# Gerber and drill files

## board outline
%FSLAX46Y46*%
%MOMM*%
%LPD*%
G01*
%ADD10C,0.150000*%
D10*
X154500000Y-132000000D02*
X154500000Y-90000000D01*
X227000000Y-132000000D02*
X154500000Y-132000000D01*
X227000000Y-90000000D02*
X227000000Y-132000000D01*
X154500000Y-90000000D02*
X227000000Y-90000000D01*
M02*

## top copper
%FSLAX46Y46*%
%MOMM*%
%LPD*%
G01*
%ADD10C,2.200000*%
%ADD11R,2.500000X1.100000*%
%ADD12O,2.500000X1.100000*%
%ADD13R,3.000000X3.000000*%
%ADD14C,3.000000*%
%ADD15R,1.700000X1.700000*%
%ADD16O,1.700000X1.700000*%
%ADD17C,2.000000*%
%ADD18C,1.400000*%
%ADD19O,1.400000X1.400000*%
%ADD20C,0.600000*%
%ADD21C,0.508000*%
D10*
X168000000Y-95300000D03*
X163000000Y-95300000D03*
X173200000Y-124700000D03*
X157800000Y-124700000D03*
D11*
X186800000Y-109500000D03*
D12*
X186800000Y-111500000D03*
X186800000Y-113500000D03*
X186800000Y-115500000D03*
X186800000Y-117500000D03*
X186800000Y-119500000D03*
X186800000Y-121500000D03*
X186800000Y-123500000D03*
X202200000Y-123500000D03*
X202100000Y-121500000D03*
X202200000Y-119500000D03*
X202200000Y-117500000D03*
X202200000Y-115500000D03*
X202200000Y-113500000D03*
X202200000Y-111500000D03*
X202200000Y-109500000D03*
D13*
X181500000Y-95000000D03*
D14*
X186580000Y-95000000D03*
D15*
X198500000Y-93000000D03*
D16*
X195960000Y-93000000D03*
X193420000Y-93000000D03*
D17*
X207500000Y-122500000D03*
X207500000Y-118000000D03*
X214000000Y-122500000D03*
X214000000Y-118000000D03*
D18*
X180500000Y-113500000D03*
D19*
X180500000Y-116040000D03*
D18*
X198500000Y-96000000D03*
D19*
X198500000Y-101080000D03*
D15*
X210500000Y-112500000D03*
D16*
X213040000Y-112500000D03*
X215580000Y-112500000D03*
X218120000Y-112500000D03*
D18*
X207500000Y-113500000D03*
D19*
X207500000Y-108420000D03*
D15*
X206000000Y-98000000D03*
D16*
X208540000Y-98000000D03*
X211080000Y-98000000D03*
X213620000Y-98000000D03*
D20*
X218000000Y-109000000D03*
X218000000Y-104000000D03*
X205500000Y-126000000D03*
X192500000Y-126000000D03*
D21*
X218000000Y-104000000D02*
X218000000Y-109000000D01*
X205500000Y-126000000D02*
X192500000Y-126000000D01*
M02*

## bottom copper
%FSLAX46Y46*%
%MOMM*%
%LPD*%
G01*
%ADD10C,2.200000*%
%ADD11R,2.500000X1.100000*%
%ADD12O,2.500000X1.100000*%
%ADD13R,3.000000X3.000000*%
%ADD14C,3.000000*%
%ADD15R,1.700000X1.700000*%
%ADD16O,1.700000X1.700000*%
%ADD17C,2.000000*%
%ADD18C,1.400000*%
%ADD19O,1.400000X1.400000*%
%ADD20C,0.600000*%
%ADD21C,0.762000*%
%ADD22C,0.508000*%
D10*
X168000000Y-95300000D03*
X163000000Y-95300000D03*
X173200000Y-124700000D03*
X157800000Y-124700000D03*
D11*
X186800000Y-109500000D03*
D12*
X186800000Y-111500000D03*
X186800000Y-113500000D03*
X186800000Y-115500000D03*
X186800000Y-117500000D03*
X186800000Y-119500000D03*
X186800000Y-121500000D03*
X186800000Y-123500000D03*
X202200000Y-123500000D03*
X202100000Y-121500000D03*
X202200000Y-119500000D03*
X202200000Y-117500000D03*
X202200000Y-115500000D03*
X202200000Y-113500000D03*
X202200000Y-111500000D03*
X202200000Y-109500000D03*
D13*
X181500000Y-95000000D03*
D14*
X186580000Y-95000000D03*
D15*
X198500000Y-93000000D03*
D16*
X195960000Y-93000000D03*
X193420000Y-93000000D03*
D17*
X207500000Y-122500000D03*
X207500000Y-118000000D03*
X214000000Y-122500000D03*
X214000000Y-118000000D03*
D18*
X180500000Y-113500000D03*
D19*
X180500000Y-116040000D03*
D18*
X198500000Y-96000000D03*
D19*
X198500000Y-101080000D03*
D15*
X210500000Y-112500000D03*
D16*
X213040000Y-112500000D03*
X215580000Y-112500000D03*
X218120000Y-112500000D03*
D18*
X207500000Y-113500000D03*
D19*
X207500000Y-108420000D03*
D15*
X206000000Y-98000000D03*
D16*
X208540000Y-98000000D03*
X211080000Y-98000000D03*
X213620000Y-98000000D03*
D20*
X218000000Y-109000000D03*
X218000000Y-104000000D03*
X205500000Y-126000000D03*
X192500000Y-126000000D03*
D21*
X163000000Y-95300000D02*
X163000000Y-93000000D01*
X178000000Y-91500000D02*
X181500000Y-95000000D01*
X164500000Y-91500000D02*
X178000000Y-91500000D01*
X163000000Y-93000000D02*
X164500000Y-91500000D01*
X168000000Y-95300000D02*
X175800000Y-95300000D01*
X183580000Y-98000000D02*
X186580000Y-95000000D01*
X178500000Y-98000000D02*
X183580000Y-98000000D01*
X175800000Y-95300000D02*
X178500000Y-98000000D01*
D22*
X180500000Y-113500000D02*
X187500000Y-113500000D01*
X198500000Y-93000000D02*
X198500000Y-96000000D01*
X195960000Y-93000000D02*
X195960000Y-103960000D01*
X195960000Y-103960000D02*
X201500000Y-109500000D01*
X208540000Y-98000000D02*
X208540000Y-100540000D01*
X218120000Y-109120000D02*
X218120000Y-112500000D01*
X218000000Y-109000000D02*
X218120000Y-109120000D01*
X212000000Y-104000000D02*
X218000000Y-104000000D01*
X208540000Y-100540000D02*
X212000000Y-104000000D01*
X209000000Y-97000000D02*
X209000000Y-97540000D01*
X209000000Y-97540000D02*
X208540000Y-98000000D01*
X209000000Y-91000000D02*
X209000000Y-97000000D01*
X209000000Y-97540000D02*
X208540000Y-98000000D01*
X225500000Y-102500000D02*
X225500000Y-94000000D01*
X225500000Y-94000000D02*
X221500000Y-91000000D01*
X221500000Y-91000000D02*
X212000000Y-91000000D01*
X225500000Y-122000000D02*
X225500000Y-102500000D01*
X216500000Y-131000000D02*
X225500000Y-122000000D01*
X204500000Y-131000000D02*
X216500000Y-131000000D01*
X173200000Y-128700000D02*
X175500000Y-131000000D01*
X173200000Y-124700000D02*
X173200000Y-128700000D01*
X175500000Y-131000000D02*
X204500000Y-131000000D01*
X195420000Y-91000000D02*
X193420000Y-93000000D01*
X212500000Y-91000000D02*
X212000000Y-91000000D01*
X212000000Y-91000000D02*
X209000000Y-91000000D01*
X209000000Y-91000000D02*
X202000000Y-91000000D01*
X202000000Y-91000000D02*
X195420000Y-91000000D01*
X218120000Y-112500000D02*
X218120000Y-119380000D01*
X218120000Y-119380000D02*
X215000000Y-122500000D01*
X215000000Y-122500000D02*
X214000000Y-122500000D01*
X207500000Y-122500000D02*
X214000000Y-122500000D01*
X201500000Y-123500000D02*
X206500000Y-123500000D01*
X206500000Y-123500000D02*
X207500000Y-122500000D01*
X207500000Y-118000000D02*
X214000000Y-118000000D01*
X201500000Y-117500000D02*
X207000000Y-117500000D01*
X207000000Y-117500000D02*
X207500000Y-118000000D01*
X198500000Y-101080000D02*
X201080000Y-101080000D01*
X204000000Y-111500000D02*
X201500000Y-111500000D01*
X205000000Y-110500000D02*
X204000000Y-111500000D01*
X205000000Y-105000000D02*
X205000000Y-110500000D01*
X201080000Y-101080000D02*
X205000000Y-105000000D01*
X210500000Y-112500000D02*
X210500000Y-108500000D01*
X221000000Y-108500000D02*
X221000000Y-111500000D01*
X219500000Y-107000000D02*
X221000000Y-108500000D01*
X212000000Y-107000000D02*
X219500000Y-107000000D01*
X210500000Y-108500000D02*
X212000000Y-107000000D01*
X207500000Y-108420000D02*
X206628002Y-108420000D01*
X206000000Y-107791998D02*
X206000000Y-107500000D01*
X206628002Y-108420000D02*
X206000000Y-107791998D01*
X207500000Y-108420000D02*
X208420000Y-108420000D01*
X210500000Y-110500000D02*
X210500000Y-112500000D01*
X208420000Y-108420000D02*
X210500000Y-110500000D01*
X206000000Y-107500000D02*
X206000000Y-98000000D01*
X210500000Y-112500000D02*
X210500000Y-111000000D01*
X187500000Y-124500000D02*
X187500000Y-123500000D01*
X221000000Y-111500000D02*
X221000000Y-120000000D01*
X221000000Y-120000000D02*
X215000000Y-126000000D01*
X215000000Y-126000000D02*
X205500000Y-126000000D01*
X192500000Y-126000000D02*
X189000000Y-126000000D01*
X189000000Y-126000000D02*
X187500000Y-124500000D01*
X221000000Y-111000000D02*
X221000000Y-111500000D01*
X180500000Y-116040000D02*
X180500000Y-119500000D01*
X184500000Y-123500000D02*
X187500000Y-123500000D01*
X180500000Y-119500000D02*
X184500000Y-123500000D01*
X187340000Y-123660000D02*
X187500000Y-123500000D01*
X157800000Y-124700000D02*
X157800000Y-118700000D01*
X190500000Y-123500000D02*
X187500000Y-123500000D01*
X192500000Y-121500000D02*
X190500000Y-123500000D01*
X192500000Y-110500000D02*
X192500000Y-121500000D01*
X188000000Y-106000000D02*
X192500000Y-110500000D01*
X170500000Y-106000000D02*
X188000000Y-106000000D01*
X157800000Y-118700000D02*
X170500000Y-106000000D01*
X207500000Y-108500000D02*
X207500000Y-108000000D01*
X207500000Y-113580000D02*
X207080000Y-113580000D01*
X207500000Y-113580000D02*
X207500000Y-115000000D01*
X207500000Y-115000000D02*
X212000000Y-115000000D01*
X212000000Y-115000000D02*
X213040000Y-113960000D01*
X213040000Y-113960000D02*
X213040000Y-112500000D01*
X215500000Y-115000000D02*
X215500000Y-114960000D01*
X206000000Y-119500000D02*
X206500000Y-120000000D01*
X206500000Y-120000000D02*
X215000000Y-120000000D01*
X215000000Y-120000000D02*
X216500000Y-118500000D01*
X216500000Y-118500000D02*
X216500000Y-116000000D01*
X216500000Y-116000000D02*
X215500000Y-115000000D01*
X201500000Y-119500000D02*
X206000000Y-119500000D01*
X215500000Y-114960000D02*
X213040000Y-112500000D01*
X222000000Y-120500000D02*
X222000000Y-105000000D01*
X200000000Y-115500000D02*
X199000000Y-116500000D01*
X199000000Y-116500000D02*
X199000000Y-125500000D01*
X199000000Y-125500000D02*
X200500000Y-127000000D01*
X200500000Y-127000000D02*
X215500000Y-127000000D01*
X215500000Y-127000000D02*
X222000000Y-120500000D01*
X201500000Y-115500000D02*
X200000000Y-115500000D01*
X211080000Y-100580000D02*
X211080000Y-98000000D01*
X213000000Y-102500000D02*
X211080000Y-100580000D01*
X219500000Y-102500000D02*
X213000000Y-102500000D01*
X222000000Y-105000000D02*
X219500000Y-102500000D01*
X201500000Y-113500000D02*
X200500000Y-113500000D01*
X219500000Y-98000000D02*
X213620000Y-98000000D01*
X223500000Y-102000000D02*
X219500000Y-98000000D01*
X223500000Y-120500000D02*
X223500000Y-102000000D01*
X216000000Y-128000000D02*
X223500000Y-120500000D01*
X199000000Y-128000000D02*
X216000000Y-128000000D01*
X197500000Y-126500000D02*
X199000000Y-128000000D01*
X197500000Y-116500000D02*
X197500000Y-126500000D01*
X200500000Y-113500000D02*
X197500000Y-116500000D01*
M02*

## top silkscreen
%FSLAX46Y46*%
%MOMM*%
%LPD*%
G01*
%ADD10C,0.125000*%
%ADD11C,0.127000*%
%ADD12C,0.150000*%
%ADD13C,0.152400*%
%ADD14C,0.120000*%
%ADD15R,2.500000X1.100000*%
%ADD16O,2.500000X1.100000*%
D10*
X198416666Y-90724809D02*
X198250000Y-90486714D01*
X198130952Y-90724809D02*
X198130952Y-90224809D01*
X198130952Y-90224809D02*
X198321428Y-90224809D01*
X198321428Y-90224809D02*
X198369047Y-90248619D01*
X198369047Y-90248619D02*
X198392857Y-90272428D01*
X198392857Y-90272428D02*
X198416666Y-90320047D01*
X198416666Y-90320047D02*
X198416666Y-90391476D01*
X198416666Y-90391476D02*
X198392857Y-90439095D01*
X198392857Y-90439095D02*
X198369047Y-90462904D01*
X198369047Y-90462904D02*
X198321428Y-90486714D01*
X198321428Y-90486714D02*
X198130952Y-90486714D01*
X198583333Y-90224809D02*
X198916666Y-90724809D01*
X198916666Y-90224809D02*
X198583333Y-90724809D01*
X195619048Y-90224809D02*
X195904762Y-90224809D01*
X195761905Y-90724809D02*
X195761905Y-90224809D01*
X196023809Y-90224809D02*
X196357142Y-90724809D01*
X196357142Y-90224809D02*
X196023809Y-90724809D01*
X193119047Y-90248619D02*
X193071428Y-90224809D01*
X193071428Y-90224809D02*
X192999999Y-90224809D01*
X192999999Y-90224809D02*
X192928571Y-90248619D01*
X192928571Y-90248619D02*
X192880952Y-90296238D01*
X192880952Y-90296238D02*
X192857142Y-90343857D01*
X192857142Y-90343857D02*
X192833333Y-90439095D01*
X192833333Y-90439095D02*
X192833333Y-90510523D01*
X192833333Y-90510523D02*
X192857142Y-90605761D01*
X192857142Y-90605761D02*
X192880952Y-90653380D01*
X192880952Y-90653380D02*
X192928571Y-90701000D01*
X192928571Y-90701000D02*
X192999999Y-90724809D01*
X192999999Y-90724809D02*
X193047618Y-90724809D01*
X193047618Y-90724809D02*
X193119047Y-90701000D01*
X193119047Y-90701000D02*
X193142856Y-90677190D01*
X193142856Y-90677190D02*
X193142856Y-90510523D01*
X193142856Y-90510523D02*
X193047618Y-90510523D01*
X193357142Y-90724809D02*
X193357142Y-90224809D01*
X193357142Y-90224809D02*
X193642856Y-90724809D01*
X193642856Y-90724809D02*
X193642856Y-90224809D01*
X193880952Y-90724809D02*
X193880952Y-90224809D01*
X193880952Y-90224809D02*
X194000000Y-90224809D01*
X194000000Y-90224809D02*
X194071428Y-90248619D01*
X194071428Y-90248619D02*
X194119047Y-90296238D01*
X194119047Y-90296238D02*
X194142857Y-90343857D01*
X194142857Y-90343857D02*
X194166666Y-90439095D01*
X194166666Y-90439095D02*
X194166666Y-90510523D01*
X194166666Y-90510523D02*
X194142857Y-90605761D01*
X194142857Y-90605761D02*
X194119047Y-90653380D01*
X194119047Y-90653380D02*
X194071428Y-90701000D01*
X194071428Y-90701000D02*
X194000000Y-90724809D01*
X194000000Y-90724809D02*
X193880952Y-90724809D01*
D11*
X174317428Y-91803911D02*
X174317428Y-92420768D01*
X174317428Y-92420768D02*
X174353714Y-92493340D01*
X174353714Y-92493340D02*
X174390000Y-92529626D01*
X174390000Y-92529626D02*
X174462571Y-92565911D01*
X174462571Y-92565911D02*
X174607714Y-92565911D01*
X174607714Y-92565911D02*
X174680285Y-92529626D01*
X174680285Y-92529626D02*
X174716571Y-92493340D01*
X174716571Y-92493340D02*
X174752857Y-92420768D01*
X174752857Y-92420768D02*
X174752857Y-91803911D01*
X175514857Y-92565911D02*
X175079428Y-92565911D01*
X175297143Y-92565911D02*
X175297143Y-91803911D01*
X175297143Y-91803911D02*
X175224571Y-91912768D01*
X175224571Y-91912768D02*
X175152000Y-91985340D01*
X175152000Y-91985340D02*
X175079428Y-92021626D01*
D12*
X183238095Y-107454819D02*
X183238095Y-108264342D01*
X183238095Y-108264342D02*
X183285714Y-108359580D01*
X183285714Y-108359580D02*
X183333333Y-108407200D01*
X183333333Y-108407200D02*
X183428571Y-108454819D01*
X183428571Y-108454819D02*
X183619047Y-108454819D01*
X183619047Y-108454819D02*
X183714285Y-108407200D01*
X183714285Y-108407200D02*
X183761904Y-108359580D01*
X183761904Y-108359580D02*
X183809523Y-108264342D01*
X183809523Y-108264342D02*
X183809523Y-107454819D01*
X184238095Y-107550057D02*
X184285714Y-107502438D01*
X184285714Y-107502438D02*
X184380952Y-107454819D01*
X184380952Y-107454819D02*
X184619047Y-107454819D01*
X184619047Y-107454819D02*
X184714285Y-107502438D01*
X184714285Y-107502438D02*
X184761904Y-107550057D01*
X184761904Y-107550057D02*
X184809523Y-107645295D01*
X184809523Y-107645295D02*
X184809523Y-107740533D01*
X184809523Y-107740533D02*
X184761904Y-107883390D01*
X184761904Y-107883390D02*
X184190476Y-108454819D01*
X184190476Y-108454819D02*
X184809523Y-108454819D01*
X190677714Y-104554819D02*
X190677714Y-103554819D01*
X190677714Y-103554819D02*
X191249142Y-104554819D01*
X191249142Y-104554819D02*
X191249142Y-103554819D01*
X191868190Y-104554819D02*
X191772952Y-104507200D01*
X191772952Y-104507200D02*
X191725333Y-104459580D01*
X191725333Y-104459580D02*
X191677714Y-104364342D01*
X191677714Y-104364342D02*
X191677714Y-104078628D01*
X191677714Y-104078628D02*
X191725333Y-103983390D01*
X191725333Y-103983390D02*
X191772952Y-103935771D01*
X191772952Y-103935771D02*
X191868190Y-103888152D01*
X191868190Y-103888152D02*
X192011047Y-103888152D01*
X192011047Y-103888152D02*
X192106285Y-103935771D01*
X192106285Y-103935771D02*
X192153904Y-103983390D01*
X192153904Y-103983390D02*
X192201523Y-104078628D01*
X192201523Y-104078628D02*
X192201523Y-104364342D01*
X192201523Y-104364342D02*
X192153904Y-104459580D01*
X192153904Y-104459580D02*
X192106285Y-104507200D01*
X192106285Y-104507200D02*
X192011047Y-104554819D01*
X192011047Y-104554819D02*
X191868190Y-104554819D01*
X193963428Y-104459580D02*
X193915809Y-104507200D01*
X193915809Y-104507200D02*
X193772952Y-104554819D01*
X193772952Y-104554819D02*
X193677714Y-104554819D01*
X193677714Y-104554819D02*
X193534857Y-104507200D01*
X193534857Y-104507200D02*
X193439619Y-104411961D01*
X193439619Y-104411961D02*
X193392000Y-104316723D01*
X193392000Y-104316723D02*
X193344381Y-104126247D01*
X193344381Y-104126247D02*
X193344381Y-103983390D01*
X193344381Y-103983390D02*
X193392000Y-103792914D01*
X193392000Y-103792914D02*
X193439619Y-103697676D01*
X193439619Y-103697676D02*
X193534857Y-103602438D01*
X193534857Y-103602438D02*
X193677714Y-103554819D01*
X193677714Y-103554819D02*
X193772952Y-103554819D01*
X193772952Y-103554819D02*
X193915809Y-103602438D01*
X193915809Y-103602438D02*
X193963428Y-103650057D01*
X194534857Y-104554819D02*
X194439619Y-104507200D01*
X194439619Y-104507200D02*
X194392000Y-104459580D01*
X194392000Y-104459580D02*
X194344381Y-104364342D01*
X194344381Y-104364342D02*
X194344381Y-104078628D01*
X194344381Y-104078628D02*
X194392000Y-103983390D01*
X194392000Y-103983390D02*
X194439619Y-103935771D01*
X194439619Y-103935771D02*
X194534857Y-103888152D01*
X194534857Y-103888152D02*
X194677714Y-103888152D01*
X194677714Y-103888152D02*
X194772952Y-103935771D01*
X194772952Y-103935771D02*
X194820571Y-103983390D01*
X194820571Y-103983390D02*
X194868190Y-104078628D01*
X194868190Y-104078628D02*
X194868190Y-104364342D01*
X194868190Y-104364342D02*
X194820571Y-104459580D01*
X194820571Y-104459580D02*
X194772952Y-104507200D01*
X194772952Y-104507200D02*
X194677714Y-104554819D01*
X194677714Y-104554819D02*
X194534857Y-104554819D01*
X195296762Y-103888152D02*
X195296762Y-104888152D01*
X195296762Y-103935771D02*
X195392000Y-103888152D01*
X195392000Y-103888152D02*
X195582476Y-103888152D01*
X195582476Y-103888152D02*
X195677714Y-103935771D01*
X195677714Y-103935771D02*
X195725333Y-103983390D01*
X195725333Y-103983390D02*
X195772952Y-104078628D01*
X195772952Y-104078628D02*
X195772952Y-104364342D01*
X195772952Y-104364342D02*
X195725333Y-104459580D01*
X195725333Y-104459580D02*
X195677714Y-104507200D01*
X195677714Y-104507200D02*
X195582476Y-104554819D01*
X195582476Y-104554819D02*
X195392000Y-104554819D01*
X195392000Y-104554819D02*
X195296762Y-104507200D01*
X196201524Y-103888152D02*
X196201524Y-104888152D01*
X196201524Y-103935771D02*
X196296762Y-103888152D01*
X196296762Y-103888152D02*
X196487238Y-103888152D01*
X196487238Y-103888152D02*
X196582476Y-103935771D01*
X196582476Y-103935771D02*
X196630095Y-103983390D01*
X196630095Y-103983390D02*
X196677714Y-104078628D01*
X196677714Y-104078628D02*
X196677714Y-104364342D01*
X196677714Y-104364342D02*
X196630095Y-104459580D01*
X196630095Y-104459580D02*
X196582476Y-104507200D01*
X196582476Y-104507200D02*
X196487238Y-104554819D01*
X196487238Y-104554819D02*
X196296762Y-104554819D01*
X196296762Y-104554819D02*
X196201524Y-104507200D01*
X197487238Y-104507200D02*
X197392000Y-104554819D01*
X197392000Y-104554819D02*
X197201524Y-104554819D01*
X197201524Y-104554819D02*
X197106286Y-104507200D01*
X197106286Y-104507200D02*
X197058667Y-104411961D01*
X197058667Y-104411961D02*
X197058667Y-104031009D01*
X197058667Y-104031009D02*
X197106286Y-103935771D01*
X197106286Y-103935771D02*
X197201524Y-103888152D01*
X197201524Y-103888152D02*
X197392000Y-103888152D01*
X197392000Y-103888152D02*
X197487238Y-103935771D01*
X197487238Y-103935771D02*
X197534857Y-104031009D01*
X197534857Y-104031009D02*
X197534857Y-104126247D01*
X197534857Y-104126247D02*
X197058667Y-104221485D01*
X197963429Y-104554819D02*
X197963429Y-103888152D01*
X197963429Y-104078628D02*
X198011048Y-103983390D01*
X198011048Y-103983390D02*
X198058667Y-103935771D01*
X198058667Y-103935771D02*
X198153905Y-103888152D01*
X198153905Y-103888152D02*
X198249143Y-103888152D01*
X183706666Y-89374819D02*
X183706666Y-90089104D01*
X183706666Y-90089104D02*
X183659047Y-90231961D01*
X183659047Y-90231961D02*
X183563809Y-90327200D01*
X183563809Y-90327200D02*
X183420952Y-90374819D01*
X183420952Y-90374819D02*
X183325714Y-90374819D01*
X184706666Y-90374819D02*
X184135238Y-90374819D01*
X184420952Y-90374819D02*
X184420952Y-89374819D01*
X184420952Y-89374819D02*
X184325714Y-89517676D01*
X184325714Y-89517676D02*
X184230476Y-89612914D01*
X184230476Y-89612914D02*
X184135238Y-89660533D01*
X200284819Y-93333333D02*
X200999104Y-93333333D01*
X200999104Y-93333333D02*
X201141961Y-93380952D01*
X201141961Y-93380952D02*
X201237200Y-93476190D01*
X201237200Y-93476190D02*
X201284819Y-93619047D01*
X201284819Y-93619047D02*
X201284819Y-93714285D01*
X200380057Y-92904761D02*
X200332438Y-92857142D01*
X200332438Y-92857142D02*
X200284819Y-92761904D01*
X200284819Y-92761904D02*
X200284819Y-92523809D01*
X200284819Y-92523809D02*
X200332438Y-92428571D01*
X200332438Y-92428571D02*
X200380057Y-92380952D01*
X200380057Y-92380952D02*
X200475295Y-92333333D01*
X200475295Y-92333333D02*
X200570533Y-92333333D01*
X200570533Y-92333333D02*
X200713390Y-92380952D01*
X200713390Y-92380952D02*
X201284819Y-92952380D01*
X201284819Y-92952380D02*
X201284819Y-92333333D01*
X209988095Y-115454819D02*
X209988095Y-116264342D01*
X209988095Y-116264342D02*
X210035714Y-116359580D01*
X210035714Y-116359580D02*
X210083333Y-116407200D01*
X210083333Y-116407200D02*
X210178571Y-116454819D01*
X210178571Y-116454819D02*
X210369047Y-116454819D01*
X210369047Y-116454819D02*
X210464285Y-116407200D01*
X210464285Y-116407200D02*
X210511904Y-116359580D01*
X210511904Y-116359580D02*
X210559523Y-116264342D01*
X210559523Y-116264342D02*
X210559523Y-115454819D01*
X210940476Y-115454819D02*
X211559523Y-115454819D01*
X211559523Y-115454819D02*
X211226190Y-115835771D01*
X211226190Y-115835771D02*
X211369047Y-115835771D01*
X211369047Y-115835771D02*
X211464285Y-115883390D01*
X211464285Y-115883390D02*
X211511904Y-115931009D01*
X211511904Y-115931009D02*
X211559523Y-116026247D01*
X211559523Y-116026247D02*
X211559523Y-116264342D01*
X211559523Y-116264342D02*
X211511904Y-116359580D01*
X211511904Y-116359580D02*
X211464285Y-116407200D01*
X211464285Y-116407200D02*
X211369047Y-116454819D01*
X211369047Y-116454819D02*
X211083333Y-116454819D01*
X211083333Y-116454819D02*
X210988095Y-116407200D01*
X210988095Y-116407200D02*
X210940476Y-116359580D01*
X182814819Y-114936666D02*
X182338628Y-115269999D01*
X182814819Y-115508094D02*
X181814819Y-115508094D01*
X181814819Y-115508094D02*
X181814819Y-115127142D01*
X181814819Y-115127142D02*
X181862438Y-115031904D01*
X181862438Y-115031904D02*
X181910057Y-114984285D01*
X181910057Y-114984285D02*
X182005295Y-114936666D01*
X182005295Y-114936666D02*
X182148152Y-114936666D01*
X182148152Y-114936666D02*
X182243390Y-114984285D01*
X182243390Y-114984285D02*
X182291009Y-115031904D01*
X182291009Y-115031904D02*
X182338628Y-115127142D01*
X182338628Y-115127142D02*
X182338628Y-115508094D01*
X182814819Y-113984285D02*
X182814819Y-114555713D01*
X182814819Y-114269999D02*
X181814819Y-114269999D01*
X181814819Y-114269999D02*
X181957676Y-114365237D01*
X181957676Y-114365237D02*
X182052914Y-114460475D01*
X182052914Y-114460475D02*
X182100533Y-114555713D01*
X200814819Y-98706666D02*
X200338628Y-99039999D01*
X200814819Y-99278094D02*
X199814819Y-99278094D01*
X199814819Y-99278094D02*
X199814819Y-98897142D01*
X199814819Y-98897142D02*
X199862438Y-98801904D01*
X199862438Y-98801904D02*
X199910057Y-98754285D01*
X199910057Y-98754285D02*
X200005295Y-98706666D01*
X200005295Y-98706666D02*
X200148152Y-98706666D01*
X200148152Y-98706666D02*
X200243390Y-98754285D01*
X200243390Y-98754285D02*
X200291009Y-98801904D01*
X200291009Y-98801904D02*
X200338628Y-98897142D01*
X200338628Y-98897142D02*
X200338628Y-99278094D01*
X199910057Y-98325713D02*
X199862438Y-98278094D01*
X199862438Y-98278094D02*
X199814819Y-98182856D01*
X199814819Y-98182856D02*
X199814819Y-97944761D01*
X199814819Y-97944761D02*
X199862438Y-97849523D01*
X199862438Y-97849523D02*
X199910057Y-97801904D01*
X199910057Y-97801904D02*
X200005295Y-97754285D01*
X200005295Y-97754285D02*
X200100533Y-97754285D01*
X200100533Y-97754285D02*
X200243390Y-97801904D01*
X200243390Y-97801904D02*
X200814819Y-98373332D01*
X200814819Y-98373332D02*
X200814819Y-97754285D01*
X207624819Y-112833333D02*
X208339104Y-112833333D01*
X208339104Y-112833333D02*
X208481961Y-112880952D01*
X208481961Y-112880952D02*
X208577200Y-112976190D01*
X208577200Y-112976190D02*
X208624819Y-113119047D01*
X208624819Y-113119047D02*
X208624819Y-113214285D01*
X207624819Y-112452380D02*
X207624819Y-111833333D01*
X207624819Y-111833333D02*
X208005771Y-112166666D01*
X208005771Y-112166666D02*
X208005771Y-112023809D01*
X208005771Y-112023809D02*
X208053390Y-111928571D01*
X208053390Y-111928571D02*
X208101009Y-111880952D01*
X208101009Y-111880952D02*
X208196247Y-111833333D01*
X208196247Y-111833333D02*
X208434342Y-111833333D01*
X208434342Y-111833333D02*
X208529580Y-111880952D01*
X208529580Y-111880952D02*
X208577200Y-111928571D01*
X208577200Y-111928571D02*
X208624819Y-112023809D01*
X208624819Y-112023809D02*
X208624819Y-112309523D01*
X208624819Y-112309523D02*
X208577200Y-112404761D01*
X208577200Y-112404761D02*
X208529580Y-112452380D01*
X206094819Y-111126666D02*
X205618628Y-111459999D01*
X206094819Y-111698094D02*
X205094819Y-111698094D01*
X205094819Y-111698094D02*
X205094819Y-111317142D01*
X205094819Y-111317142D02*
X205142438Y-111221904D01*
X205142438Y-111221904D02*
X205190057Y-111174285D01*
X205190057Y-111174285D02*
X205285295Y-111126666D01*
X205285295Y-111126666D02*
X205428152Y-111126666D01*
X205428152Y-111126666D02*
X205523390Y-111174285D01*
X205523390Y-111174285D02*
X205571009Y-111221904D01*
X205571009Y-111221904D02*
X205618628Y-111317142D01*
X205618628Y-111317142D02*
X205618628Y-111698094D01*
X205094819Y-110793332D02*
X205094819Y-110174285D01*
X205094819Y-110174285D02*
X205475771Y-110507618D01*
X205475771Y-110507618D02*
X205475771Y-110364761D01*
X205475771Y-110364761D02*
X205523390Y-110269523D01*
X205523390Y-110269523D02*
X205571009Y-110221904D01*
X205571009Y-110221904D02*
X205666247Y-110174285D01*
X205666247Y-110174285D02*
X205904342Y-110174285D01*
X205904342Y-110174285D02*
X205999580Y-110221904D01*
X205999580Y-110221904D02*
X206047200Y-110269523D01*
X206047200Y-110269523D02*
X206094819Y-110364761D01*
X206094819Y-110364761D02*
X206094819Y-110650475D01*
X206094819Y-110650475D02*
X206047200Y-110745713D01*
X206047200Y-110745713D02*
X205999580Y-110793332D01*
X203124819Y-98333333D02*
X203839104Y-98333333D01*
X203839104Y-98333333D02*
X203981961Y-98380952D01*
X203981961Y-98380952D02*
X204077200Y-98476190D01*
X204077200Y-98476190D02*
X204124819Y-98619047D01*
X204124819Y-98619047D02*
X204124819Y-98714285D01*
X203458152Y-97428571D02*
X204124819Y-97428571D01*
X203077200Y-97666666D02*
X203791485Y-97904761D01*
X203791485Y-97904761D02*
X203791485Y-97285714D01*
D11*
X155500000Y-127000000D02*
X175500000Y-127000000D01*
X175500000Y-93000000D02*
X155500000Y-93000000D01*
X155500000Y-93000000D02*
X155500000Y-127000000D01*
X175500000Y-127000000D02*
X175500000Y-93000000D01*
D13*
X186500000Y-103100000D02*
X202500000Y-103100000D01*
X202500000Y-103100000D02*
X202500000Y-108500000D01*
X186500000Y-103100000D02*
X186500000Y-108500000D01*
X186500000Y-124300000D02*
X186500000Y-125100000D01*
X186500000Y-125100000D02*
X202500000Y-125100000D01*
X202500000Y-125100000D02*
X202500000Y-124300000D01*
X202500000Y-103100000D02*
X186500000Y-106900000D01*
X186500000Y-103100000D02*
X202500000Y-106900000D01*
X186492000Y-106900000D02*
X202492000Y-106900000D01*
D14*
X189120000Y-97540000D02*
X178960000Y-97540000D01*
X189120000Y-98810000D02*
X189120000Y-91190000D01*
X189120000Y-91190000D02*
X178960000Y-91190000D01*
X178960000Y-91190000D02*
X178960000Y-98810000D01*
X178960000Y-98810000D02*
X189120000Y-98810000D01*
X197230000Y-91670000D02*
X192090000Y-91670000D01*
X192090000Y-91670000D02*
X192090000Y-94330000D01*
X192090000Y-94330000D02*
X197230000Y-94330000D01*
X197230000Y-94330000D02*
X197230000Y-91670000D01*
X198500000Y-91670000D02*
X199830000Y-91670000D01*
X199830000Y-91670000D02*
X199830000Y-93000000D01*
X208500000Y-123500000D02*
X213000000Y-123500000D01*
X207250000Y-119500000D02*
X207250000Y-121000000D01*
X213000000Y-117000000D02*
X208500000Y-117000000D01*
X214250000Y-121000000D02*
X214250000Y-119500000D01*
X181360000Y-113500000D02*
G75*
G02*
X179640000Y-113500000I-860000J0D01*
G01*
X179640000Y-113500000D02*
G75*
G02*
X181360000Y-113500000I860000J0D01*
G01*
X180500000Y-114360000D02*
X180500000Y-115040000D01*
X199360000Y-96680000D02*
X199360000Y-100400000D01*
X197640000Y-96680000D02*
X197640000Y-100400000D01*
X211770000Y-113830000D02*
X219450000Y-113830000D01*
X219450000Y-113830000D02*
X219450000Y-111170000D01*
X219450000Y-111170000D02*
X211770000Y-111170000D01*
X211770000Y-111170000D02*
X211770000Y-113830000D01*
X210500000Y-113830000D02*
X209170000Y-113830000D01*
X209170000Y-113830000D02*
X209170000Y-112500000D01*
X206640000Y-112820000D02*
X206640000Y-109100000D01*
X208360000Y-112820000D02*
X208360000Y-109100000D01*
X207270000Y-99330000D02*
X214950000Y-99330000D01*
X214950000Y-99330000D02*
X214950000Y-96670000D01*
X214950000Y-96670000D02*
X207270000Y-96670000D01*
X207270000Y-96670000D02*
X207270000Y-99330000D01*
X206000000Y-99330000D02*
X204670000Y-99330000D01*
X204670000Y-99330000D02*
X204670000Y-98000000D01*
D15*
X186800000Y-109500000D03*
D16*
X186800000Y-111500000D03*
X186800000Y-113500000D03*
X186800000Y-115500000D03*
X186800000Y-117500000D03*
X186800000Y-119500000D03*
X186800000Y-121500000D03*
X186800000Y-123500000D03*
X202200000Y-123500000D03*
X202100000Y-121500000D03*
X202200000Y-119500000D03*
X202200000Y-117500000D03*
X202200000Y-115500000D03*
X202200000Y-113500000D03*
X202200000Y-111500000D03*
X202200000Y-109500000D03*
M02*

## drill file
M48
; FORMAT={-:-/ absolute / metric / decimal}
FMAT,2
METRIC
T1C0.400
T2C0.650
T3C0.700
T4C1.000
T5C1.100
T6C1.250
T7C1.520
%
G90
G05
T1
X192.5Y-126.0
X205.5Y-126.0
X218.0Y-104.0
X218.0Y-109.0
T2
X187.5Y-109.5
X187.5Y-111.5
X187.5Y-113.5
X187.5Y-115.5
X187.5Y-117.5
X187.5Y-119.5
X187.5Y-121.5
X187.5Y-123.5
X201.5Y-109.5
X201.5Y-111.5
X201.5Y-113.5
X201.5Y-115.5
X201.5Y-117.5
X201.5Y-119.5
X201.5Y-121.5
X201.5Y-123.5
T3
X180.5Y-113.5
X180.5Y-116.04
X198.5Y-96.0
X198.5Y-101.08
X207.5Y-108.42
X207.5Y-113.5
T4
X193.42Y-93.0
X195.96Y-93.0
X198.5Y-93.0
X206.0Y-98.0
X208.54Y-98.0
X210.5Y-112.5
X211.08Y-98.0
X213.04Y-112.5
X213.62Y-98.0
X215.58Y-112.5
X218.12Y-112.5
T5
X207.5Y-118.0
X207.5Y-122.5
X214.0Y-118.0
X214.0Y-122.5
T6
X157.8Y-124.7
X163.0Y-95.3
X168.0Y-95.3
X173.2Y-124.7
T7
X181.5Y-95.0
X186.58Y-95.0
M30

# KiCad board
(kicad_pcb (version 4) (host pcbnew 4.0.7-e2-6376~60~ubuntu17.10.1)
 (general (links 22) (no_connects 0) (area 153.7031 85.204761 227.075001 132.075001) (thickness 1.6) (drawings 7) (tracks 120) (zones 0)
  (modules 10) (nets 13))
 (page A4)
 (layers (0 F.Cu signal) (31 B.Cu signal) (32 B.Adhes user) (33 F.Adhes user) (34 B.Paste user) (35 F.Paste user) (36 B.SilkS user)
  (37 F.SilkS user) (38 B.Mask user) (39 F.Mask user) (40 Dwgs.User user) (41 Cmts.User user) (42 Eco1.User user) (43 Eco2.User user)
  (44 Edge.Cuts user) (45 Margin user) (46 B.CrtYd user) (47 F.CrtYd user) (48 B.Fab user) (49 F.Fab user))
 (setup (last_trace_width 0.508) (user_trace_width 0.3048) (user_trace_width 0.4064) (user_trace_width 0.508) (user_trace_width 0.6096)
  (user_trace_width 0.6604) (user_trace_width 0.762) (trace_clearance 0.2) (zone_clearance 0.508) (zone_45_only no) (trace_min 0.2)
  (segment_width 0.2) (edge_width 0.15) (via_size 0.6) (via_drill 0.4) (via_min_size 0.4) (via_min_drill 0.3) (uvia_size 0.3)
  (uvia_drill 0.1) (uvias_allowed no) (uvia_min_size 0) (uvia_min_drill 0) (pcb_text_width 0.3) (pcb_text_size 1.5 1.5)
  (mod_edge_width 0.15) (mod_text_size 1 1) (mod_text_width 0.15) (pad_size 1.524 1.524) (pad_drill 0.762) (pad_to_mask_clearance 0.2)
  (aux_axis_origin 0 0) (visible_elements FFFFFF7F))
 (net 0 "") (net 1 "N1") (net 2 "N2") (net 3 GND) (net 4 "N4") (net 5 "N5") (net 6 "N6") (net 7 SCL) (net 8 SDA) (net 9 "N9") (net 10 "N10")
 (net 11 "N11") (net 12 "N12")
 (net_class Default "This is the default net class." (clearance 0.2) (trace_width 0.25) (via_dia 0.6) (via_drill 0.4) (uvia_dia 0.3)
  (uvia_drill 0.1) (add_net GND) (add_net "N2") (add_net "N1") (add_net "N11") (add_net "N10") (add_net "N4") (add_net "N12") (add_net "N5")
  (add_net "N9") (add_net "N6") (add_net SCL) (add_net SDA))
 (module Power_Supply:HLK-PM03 (layer F.Cu) (at 165.5 110 270)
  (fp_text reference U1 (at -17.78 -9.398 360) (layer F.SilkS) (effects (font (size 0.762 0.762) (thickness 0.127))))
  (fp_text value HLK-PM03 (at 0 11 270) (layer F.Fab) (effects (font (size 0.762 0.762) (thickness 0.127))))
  (fp_line (start 17 10) (end 17 -10) (layer F.SilkS) (width 0.127))
  (fp_line (start -17 -10) (end -17 10) (layer F.SilkS) (width 0.127))
  (fp_line (start -17 10) (end 17 10) (layer F.SilkS) (width 0.127))
  (fp_line (start 17 -10) (end -17 -10) (layer F.SilkS) (width 0.127))
  (pad 1 thru_hole circle (at -14.7 -2.5 270) (size 2.2 2.2) (drill 1.25) (layers *.Cu *.Mask) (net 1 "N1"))
  (pad 2 thru_hole circle (at -14.7 2.5 270) (size 2.2 2.2) (drill 1.25) (layers *.Cu *.Mask) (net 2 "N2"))
  (pad 3 thru_hole circle (at 14.7 -7.7 270) (size 2.2 2.2) (drill 1.25) (layers *.Cu *.Mask) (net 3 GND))
  (pad 4 thru_hole circle (at 14.7 7.7 270) (size 2.2 2.2) (drill 1.25) (layers *.Cu *.Mask) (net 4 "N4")))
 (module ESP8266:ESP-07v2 (layer F.Cu) (at 187.5 109.5)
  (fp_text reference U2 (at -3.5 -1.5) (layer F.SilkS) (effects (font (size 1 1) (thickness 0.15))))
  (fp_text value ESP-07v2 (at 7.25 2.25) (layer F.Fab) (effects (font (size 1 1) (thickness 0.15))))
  (fp_line (start -1 -6.4) (end 15 -6.4) (layer F.SilkS) (width 0.1524))
  (fp_line (start 15 -6.4) (end 15 -1) (layer F.SilkS) (width 0.1524))
  (fp_line (start -1 -6.4) (end -1 -1) (layer F.SilkS) (width 0.1524))
  (fp_line (start -1 14.8) (end -1 15.6) (layer F.SilkS) (width 0.1524))
  (fp_line (start -1 15.6) (end 15 15.6) (layer F.SilkS) (width 0.1524))
  (fp_line (start 15 15.6) (end 15 14.8) (layer F.SilkS) (width 0.1524))
  (fp_line (start 15 -6.4) (end -1 -2.6) (layer F.SilkS) (width 0.1524))
  (fp_line (start -1 -6.4) (end 15 -2.6) (layer F.SilkS) (width 0.1524))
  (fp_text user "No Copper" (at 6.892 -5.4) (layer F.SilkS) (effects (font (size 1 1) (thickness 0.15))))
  (fp_line (start -1.008 -2.6) (end 14.992 -2.6) (layer F.SilkS) (width 0.1524))
  (pad 1 thru_hole rect (at 0 0) (size 2.5 1.1) (drill 0.65 (offset -0.7 0)) (layers *.Cu *.Mask F.Paste F.SilkS))
  (pad 2 thru_hole oval (at 0 2) (size 2.5 1.1) (drill 0.65 (offset -0.7 0)) (layers *.Cu *.Mask F.Paste F.SilkS))
  (pad 3 thru_hole oval (at 0 4) (size 2.5 1.1) (drill 0.65 (offset -0.7 0)) (layers *.Cu *.Mask F.Paste F.SilkS) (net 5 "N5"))
  (pad 4 thru_hole oval (at 0 6) (size 2.5 1.1) (drill 0.65 (offset -0.7 0)) (layers *.Cu *.Mask F.Paste F.SilkS))
  (pad 5 thru_hole oval (at 0 8) (size 2.5 1.1) (drill 0.65 (offset -0.7 0)) (layers *.Cu *.Mask F.Paste F.SilkS))
  (pad 6 thru_hole oval (at 0 10) (size 2.5 1.1) (drill 0.65 (offset -0.7 0)) (layers *.Cu *.Mask F.Paste F.SilkS))
  (pad 7 thru_hole oval (at 0 12) (size 2.5 1.1) (drill 0.65 (offset -0.7 0)) (layers *.Cu *.Mask F.Paste F.SilkS))
  (pad 8 thru_hole oval (at 0 14) (size 2.5 1.1) (drill 0.65 (offset -0.7 0)) (layers *.Cu *.Mask F.Paste F.SilkS) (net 4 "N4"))
  (pad 9 thru_hole oval (at 14 14) (size 2.5 1.1) (drill 0.65 (offset 0.7 0)) (layers *.Cu *.Mask F.Paste F.SilkS) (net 3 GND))
  (pad 10 thru_hole oval (at 14 12) (size 2.5 1.1) (drill 0.65 (offset 0.6 0)) (layers *.Cu *.Mask F.Paste F.SilkS))
  (pad 11 thru_hole oval (at 14 10) (size 2.5 1.1) (drill 0.65 (offset 0.7 0)) (layers *.Cu *.Mask F.Paste F.SilkS))
  (pad 12 thru_hole oval (at 14 8) (size 2.5 1.1) (drill 0.65 (offset 0.7 0)) (layers *.Cu *.Mask F.Paste F.SilkS) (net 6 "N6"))
  (pad 13 thru_hole oval (at 14 6) (size 2.5 1.1) (drill 0.65 (offset 0.7 0)) (layers *.Cu *.Mask F.Paste F.SilkS) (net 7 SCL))
  (pad 14 thru_hole oval (at 14 4) (size 2.5 1.1) (drill 0.65 (offset 0.7 0)) (layers *.Cu *.Mask F.Paste F.SilkS) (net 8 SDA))
  (pad 15 thru_hole oval (at 14 2) (size 2.5 1.1) (drill 0.65 (offset 0.7 0)) (layers *.Cu *.Mask F.Paste F.SilkS) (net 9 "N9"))
  (pad 16 thru_hole oval (at 14 0) (size 2.5 1.1) (drill 0.65 (offset 0.7 0)) (layers *.Cu *.Mask F.Paste F.SilkS) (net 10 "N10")))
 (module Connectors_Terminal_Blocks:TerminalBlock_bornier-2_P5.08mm (layer F.Cu) (at 181.5 95)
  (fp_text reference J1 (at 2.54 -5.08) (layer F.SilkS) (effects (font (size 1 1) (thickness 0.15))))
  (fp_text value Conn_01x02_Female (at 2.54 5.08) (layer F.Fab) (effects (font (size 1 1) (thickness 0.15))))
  (fp_line (start 7.62 2.54) (end -2.54 2.54) (layer F.SilkS) (width 0.12))
  (fp_line (start 7.62 3.81) (end 7.62 -3.81) (layer F.SilkS) (width 0.12))
  (fp_line (start 7.62 -3.81) (end -2.54 -3.81) (layer F.SilkS) (width 0.12))
  (fp_line (start -2.54 -3.81) (end -2.54 3.81) (layer F.SilkS) (width 0.12))
  (fp_line (start -2.54 3.81) (end 7.62 3.81) (layer F.SilkS) (width 0.12))
  (pad 1 thru_hole rect (at 0 0) (size 3 3) (drill 1.52) (layers *.Cu *.Mask) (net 2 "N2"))
  (pad 2 thru_hole circle (at 5.08 0) (size 3 3) (drill 1.52) (layers *.Cu *.Mask) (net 1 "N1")))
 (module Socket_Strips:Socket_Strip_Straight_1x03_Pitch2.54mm (layer F.Cu) (at 198.5 93 270)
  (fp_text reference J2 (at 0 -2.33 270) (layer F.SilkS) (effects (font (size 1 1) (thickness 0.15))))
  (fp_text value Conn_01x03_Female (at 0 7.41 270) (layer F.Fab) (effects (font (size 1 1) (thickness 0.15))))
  (fp_line (start -1.33 1.27) (end -1.33 6.41) (layer F.SilkS) (width 0.12))
  (fp_line (start -1.33 6.41) (end 1.33 6.41) (layer F.SilkS) (width 0.12))
  (fp_line (start 1.33 6.41) (end 1.33 1.27) (layer F.SilkS) (width 0.12))
  (fp_line (start 1.33 1.27) (end -1.33 1.27) (layer F.SilkS) (width 0.12))
  (fp_line (start -1.33 0) (end -1.33 -1.33) (layer F.SilkS) (width 0.12))
  (fp_line (start -1.33 -1.33) (end 0 -1.33) (layer F.SilkS) (width 0.12))
  (pad 1 thru_hole rect (at 0 0 270) (size 1.7 1.7) (drill 1) (layers *.Cu *.Mask) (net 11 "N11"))
  (pad 2 thru_hole oval (at 0 2.54 270) (size 1.7 1.7) (drill 1) (layers *.Cu *.Mask) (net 10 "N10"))
  (pad 3 thru_hole oval (at 0 5.08 270) (size 1.7 1.7) (drill 1) (layers *.Cu *.Mask) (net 3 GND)))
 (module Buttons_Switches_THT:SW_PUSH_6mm (layer F.Cu) (at 207.5 118)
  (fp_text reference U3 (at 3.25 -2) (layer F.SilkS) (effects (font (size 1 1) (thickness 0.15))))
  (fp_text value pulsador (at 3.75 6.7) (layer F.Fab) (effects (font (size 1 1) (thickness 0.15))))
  (fp_line (start 1 5.5) (end 5.5 5.5) (layer F.SilkS) (width 0.12))
  (fp_line (start -0.25 1.5) (end -0.25 3) (layer F.SilkS) (width 0.12))
  (fp_line (start 5.5 -1) (end 1 -1) (layer F.SilkS) (width 0.12))
  (fp_line (start 6.75 3) (end 6.75 1.5) (layer F.SilkS) (width 0.12))
  (pad 2 thru_hole circle (at 0 4.5 90) (size 2 2) (drill 1.1) (layers *.Cu *.Mask) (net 3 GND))
  (pad 1 thru_hole circle (at 0 0 90) (size 2 2) (drill 1.1) (layers *.Cu *.Mask) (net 6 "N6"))
  (pad 2 thru_hole circle (at 6.5 4.5 90) (size 2 2) (drill 1.1) (layers *.Cu *.Mask) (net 3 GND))
  (pad 1 thru_hole circle (at 6.5 0 90) (size 2 2) (drill 1.1) (layers *.Cu *.Mask) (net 6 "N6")))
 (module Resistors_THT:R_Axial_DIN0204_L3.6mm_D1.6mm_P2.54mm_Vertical (layer F.Cu) (at 180.5 113.5 270)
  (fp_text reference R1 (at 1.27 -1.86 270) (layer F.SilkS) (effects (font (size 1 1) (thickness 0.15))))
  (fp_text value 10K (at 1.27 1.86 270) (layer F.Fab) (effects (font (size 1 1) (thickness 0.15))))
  (fp_circle (center 0 0) (end 0.86 0) (layer F.SilkS) (width 0.12))
  (fp_line (start 0.86 0) (end 1.54 0) (layer F.SilkS) (width 0.12))
  (pad 1 thru_hole circle (at 0 0 270) (size 1.4 1.4) (drill 0.7) (layers *.Cu *.Mask) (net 5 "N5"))
  (pad 2 thru_hole oval (at 2.54 0 270) (size 1.4 1.4) (drill 0.7) (layers *.Cu *.Mask) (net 4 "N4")))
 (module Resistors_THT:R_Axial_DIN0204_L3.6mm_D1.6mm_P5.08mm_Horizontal (layer F.Cu) (at 198.5 96 270)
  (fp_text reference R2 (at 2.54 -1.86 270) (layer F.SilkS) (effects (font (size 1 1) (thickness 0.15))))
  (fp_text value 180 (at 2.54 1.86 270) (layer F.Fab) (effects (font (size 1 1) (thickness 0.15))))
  (fp_line (start 0.68 -0.86) (end 4.4 -0.86) (layer F.SilkS) (width 0.12))
  (fp_line (start 0.68 0.86) (end 4.4 0.86) (layer F.SilkS) (width 0.12))
  (pad 1 thru_hole circle (at 0 0 270) (size 1.4 1.4) (drill 0.7) (layers *.Cu *.Mask) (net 11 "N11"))
  (pad 2 thru_hole oval (at 5.08 0 270) (size 1.4 1.4) (drill 0.7) (layers *.Cu *.Mask) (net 9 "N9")))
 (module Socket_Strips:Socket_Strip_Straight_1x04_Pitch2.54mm (layer F.Cu) (at 210.5 112.5 90)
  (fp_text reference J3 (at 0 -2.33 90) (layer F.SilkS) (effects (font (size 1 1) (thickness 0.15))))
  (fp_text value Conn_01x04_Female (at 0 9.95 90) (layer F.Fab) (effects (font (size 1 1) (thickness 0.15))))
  (fp_line (start -1.33 1.27) (end -1.33 8.95) (layer F.SilkS) (width 0.12))
  (fp_line (start -1.33 8.95) (end 1.33 8.95) (layer F.SilkS) (width 0.12))
  (fp_line (start 1.33 8.95) (end 1.33 1.27) (layer F.SilkS) (width 0.12))
  (fp_line (start 1.33 1.27) (end -1.33 1.27) (layer F.SilkS) (width 0.12))
  (fp_line (start -1.33 0) (end -1.33 -1.33) (layer F.SilkS) (width 0.12))
  (fp_line (start -1.33 -1.33) (end 0 -1.33) (layer F.SilkS) (width 0.12))
  (pad 1 thru_hole rect (at 0 0 90) (size 1.7 1.7) (drill 1) (layers *.Cu *.Mask) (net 4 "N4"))
  (pad 2 thru_hole oval (at 0 2.54 90) (size 1.7 1.7) (drill 1) (layers *.Cu *.Mask) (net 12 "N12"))
  (pad 3 thru_hole oval (at 0 5.08 90) (size 1.7 1.7) (drill 1) (layers *.Cu *.Mask))
  (pad 4 thru_hole oval (at 0 7.62 90) (size 1.7 1.7) (drill 1) (layers *.Cu *.Mask) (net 3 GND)))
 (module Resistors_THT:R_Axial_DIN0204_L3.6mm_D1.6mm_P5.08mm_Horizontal (layer F.Cu) (at 207.5 113.5 90)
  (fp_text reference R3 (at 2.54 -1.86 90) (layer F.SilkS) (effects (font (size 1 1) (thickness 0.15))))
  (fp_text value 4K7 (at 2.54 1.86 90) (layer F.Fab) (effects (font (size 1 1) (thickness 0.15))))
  (fp_line (start 0.68 -0.86) (end 4.4 -0.86) (layer F.SilkS) (width 0.12))
  (fp_line (start 0.68 0.86) (end 4.4 0.86) (layer F.SilkS) (width 0.12))
  (pad 1 thru_hole circle (at 0 0 90) (size 1.4 1.4) (drill 0.7) (layers *.Cu *.Mask) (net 12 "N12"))
  (pad 2 thru_hole oval (at 5.08 0 90) (size 1.4 1.4) (drill 0.7) (layers *.Cu *.Mask) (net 4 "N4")))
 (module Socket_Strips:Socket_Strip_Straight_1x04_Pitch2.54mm (layer F.Cu) (at 206 98 90)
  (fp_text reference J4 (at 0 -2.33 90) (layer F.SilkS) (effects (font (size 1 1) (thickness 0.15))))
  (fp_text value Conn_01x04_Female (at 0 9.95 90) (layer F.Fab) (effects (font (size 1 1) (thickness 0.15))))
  (fp_line (start -1.33 1.27) (end -1.33 8.95) (layer F.SilkS) (width 0.12))
  (fp_line (start -1.33 8.95) (end 1.33 8.95) (layer F.SilkS) (width 0.12))
  (fp_line (start 1.33 8.95) (end 1.33 1.27) (layer F.SilkS) (width 0.12))
  (fp_line (start 1.33 1.27) (end -1.33 1.27) (layer F.SilkS) (width 0.12))
  (fp_line (start -1.33 0) (end -1.33 -1.33) (layer F.SilkS) (width 0.12))
  (fp_line (start -1.33 -1.33) (end 0 -1.33) (layer F.SilkS) (width 0.12))
  (pad 1 thru_hole rect (at 0 0 90) (size 1.7 1.7) (drill 1) (layers *.Cu *.Mask) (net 4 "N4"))
  (pad 2 thru_hole oval (at 0 2.54 90) (size 1.7 1.7) (drill 1) (layers *.Cu *.Mask) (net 3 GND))
  (pad 3 thru_hole oval (at 0 5.08 90) (size 1.7 1.7) (drill 1) (layers *.Cu *.Mask) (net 7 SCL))
  (pad 4 thru_hole oval (at 0 7.62 90) (size 1.7 1.7) (drill 1) (layers *.Cu *.Mask) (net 8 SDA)))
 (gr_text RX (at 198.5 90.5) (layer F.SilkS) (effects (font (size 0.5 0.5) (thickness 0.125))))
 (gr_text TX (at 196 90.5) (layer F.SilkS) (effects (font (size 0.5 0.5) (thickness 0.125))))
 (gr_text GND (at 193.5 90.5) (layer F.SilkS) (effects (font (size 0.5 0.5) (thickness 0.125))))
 (gr_line (start 154.5 132) (end 154.5 90) (angle 90) (layer Edge.Cuts) (width 0.15))
 (gr_line (start 227 132) (end 154.5 132) (angle 90) (layer Edge.Cuts) (width 0.15))
 (gr_line (start 227 90) (end 227 132) (angle 90) (layer Edge.Cuts) (width 0.15))
 (gr_line (start 154.5 90) (end 227 90) (angle 90) (layer Edge.Cuts) (width 0.15))
 (segment (start 163 95.3) (end 163 93) (width 0.762) (layer B.Cu) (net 2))
 (segment (start 178 91.5) (end 181.5 95) (width 0.762) (layer B.Cu) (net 2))
 (segment (start 164.5 91.5) (end 178 91.5) (width 0.762) (layer B.Cu) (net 2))
 (segment (start 163 93) (end 164.5 91.5) (width 0.762) (layer B.Cu) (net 2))
 (segment (start 168 95.3) (end 175.8 95.3) (width 0.762) (layer B.Cu) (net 1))
 (segment (start 183.58 98) (end 186.58 95) (width 0.762) (layer B.Cu) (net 1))
 (segment (start 178.5 98) (end 183.58 98) (width 0.762) (layer B.Cu) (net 1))
 (segment (start 175.8 95.3) (end 178.5 98) (width 0.762) (layer B.Cu) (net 1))
 (segment (start 180.5 113.5) (end 187.5 113.5) (width 0.508) (layer B.Cu) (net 5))
 (segment (start 198.5 93) (end 198.5 96) (width 0.508) (layer B.Cu) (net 11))
 (segment (start 195.96 93) (end 195.96 103.96) (width 0.508) (layer B.Cu) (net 10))
 (segment (start 195.96 103.96) (end 201.5 109.5) (width 0.508) (layer B.Cu) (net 10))
 (segment (start 208.54 98) (end 208.54 100.54) (width 0.508) (layer B.Cu) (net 3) (status 400000))
 (segment (start 218.12 109.12) (end 218.12 112.5) (width 0.508) (layer B.Cu) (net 3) (status 800000))
 (segment (start 218 109) (end 218.12 109.12) (width 0.508) (layer B.Cu) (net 3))
 (via (at 218 109) (size 0.6) (drill 0.4) (layers F.Cu B.Cu) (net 3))
 (segment (start 218 104) (end 218 109) (width 0.508) (layer F.Cu) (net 3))
 (via (at 218 104) (size 0.6) (drill 0.4) (layers F.Cu B.Cu) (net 3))
 (segment (start 212 104) (end 218 104) (width 0.508) (layer B.Cu) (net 3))
 (segment (start 208.54 100.54) (end 212 104) (width 0.508) (layer B.Cu) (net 3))
 (segment (start 209 97) (end 209 97.54) (width 0.508) (layer B.Cu) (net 3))
 (segment (start 209 97.54) (end 208.54 98) (width 0.508) (layer B.Cu) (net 3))
 (segment (start 209 91) (end 209 97) (width 0.508) (layer B.Cu) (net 3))
 (segment (start 209 97.54) (end 208.54 98) (width 0.508) (layer B.Cu) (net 3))
 (segment (start 225.5 102.5) (end 225.5 94) (width 0.508) (layer B.Cu) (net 3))
 (segment (start 225.5 94) (end 221.5 91) (width 0.508) (layer B.Cu) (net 3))
 (segment (start 221.5 91) (end 212 91) (width 0.508) (layer B.Cu) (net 3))
 (segment (start 225.5 122) (end 225.5 102.5) (width 0.508) (layer B.Cu) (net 3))
 (segment (start 216.5 131) (end 225.5 122) (width 0.508) (layer B.Cu) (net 3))
 (segment (start 204.5 131) (end 216.5 131) (width 0.508) (layer B.Cu) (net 3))
 (segment (start 173.2 128.7) (end 175.5 131) (width 0.508) (layer B.Cu) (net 3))
 (segment (start 173.2 124.7) (end 173.2 128.7) (width 0.508) (layer B.Cu) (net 3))
 (segment (start 175.5 131) (end 204.5 131) (width 0.508) (layer B.Cu) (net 3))
 (segment (start 195.42 91) (end 193.42 93) (width 0.508) (layer B.Cu) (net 3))
 (segment (start 212.5 91) (end 212 91) (width 0.508) (layer B.Cu) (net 3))
 (segment (start 212 91) (end 209 91) (width 0.508) (layer B.Cu) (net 3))
 (segment (start 209 91) (end 202 91) (width 0.508) (layer B.Cu) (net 3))
 (segment (start 202 91) (end 195.42 91) (width 0.508) (layer B.Cu) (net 3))
 (segment (start 218.12 112.5) (end 218.12 119.38) (width 0.508) (layer B.Cu) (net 3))
 (segment (start 218.12 119.38) (end 215 122.5) (width 0.508) (layer B.Cu) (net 3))
 (segment (start 215 122.5) (end 214 122.5) (width 0.508) (layer B.Cu) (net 3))
 (segment (start 207.5 122.5) (end 214 122.5) (width 0.508) (layer B.Cu) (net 3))
 (segment (start 201.5 123.5) (end 206.5 123.5) (width 0.508) (layer B.Cu) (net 3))
 (segment (start 206.5 123.5) (end 207.5 122.5) (width 0.508) (layer B.Cu) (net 3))
 (segment (start 207.5 118) (end 214 118) (width 0.508) (layer B.Cu) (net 6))
 (segment (start 201.5 117.5) (end 207 117.5) (width 0.508) (layer B.Cu) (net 6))
 (segment (start 207 117.5) (end 207.5 118) (width 0.508) (layer B.Cu) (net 6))
 (segment (start 198.5 101.08) (end 201.08 101.08) (width 0.508) (layer B.Cu) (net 9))
 (segment (start 204 111.5) (end 201.5 111.5) (width 0.508) (layer B.Cu) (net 9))
 (segment (start 205 110.5) (end 204 111.5) (width 0.508) (layer B.Cu) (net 9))
 (segment (start 205 105) (end 205 110.5) (width 0.508) (layer B.Cu) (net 9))
 (segment (start 201.08 101.08) (end 205 105) (width 0.508) (layer B.Cu) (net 9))
 (segment (start 210.5 112.5) (end 210.5 108.5) (width 0.508) (layer B.Cu) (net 4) (status 400000))
 (segment (start 221 108.5) (end 221 111.5) (width 0.508) (layer B.Cu) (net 4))
 (segment (start 219.5 107) (end 221 108.5) (width 0.508) (layer B.Cu) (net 4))
 (segment (start 212 107) (end 219.5 107) (width 0.508) (layer B.Cu) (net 4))
 (segment (start 210.5 108.5) (end 212 107) (width 0.508) (layer B.Cu) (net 4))
 (segment (start 207.5 108.42) (end 206.628002 108.42) (width 0.508) (layer B.Cu) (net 4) (status 400000))
 (segment (start 206 107.791998) (end 206 107.5) (width 0.508) (layer B.Cu) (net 4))
 (segment (start 206.628002 108.42) (end 206 107.791998) (width 0.508) (layer B.Cu) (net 4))
 (segment (start 207.5 108.42) (end 208.42 108.42) (width 0.508) (layer B.Cu) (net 4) (status 400000))
 (segment (start 210.5 110.5) (end 210.5 112.5) (width 0.508) (layer B.Cu) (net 4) (status 800000))
 (segment (start 208.42 108.42) (end 210.5 110.5) (width 0.508) (layer B.Cu) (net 4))
 (segment (start 206 107.5) (end 206 98) (width 0.508) (layer B.Cu) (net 4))
 (segment (start 210.5 112.5) (end 210.5 111) (width 0.508) (layer B.Cu) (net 4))
 (segment (start 187.5 124.5) (end 187.5 123.5) (width 0.508) (layer B.Cu) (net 4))
 (segment (start 221 111.5) (end 221 120) (width 0.508) (layer B.Cu) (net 4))
 (segment (start 221 120) (end 215 126) (width 0.508) (layer B.Cu) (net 4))
 (segment (start 215 126) (end 205.5 126) (width 0.508) (layer B.Cu) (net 4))
 (via (at 205.5 126) (size 0.6) (drill 0.4) (layers F.Cu B.Cu) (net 4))
 (segment (start 205.5 126) (end 192.5 126) (width 0.508) (layer F.Cu) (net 4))
 (via (at 192.5 126) (size 0.6) (drill 0.4) (layers F.Cu B.Cu) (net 4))
 (segment (start 192.5 126) (end 189 126) (width 0.508) (layer B.Cu) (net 4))
 (segment (start 189 126) (end 187.5 124.5) (width 0.508) (layer B.Cu) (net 4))
 (segment (start 221 111) (end 221 111.5) (width 0.508) (layer B.Cu) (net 4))
 (segment (start 180.5 116.04) (end 180.5 119.5) (width 0.508) (layer B.Cu) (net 4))
 (segment (start 184.5 123.5) (end 187.5 123.5) (width 0.508) (layer B.Cu) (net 4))
 (segment (start 180.5 119.5) (end 184.5 123.5) (width 0.508) (layer B.Cu) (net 4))
 (segment (start 187.34 123.66) (end 187.5 123.5) (width 0.508) (layer B.Cu) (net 4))
 (segment (start 157.8 124.7) (end 157.8 118.7) (width 0.508) (layer B.Cu) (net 4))
 (segment (start 190.5 123.5) (end 187.5 123.5) (width 0.508) (layer B.Cu) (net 4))
 (segment (start 192.5 121.5) (end 190.5 123.5) (width 0.508) (layer B.Cu) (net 4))
 (segment (start 192.5 110.5) (end 192.5 121.5) (width 0.508) (layer B.Cu) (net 4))
 (segment (start 188 106) (end 192.5 110.5) (width 0.508) (layer B.Cu) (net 4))
 (segment (start 170.5 106) (end 188 106) (width 0.508) (layer B.Cu) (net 4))
 (segment (start 157.8 118.7) (end 170.5 106) (width 0.508) (layer B.Cu) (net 4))
 (segment (start 207.5 108.5) (end 207.5 108) (width 0.508) (layer B.Cu) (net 4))
 (segment (start 207.5 113.58) (end 207.08 113.58) (width 0.508) (layer B.Cu) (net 12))
 (segment (start 207.5 113.58) (end 207.5 115) (width 0.508) (layer B.Cu) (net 12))
 (segment (start 207.5 115) (end 212 115) (width 0.508) (layer B.Cu) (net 12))
 (segment (start 212 115) (end 213.04 113.96) (width 0.508) (layer B.Cu) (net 12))
 (segment (start 213.04 113.96) (end 213.04 112.5) (width 0.508) (layer B.Cu) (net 12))
 (segment (start 215.5 115) (end 215.5 114.96) (width 0.508) (layer B.Cu) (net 12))
 (segment (start 206 119.5) (end 206.5 120) (width 0.508) (layer B.Cu) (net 12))
 (segment (start 206.5 120) (end 215 120) (width 0.508) (layer B.Cu) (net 12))
 (segment (start 215 120) (end 216.5 118.5) (width 0.508) (layer B.Cu) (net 12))
 (segment (start 216.5 118.5) (end 216.5 116) (width 0.508) (layer B.Cu) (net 12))
 (segment (start 216.5 116) (end 215.5 115) (width 0.508) (layer B.Cu) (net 12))
 (segment (start 201.5 119.5) (end 206 119.5) (width 0.508) (layer B.Cu) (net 12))
 (segment (start 215.5 114.96) (end 213.04 112.5) (width 0.508) (layer B.Cu) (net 12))
 (segment (start 222 120.5) (end 222 105) (width 0.508) (layer B.Cu) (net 7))
 (segment (start 200 115.5) (end 199 116.5) (width 0.508) (layer B.Cu) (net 7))
 (segment (start 199 116.5) (end 199 125.5) (width 0.508) (layer B.Cu) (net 7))
 (segment (start 199 125.5) (end 200.5 127) (width 0.508) (layer B.Cu) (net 7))
 (segment (start 200.5 127) (end 215.5 127) (width 0.508) (layer B.Cu) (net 7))
 (segment (start 215.5 127) (end 222 120.5) (width 0.508) (layer B.Cu) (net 7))
 (segment (start 201.5 115.5) (end 200 115.5) (width 0.508) (layer B.Cu) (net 7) (status 400000))
 (segment (start 211.08 100.58) (end 211.08 98) (width 0.508) (layer B.Cu) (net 7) (status 800000))
 (segment (start 213 102.5) (end 211.08 100.58) (width 0.508) (layer B.Cu) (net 7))
 (segment (start 219.5 102.5) (end 213 102.5) (width 0.508) (layer B.Cu) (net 7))
 (segment (start 222 105) (end 219.5 102.5) (width 0.508) (layer B.Cu) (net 7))
 (segment (start 201.5 113.5) (end 200.5 113.5) (width 0.508) (layer B.Cu) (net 8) (status 400000))
 (segment (start 219.5 98) (end 213.62 98) (width 0.508) (layer B.Cu) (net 8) (status 800000))
 (segment (start 223.5 102) (end 219.5 98) (width 0.508) (layer B.Cu) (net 8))
 (segment (start 223.5 120.5) (end 223.5 102) (width 0.508) (layer B.Cu) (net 8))
 (segment (start 216 128) (end 223.5 120.5) (width 0.508) (layer B.Cu) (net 8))
 (segment (start 199 128) (end 216 128) (width 0.508) (layer B.Cu) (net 8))
 (segment (start 197.5 126.5) (end 199 128) (width 0.508) (layer B.Cu) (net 8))
 (segment (start 197.5 116.5) (end 197.5 126.5) (width 0.508) (layer B.Cu) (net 8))
 (segment (start 200.5 113.5) (end 197.5 116.5) (width 0.508) (layer B.Cu) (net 8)))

